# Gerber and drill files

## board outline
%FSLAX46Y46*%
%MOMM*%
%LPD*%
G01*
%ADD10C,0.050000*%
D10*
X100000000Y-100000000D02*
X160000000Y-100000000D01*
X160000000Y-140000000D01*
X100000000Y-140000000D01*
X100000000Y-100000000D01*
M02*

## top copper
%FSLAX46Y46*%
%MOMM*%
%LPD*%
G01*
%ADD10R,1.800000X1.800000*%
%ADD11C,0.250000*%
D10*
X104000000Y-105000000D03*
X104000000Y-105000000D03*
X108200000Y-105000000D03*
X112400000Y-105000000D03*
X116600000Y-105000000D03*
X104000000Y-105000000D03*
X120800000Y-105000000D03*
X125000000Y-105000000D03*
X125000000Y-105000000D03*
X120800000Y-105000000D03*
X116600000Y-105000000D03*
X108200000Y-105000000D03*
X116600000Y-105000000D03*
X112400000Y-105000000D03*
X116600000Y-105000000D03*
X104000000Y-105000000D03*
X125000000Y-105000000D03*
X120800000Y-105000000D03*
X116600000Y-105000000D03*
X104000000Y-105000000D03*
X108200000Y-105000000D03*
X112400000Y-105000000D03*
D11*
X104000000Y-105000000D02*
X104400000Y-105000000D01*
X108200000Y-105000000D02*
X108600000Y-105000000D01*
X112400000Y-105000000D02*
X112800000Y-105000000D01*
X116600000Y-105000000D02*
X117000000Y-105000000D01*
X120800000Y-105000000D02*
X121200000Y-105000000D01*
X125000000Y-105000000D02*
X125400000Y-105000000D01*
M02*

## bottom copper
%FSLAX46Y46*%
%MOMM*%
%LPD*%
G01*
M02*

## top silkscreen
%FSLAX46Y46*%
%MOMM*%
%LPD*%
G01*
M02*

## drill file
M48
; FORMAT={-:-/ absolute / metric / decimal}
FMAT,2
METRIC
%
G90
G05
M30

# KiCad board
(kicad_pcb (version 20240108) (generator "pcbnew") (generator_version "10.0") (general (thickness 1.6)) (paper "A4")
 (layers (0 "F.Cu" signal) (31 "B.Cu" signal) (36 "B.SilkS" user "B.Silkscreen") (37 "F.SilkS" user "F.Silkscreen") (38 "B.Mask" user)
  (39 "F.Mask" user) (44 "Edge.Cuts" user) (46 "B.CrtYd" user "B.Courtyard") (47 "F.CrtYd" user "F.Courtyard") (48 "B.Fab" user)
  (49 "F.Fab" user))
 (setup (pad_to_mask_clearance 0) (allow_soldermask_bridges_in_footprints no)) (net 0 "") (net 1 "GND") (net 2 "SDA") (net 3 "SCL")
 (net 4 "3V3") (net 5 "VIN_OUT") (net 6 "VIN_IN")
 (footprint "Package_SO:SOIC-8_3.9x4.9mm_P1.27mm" (layer "F.Cu") (at 100 100)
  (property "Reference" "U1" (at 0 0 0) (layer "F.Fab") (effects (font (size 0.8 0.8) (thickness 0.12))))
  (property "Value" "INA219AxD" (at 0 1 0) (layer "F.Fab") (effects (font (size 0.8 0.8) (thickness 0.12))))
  (pad "1" smd rect (at 4.000 5.000) (size 1.8 1.8) (layers "F.Cu" "F.Paste" "F.Mask") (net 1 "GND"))
  (pad "2" smd rect (at 4.000 5.000) (size 1.8 1.8) (layers "F.Cu" "F.Paste" "F.Mask") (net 1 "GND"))
  (pad "3" smd rect (at 8.200 5.000) (size 1.8 1.8) (layers "F.Cu" "F.Paste" "F.Mask") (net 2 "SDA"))
  (pad "4" smd rect (at 12.400 5.000) (size 1.8 1.8) (layers "F.Cu" "F.Paste" "F.Mask") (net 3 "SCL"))
  (pad "5" smd rect (at 16.600 5.000) (size 1.8 1.8) (layers "F.Cu" "F.Paste" "F.Mask") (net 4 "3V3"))
  (pad "6" smd rect (at 4.000 5.000) (size 1.8 1.8) (layers "F.Cu" "F.Paste" "F.Mask") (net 1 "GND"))
  (pad "7" smd rect (at 20.800 5.000) (size 1.8 1.8) (layers "F.Cu" "F.Paste" "F.Mask") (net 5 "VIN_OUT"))
  (pad "8" smd rect (at 25.000 5.000) (size 1.8 1.8) (layers "F.Cu" "F.Paste" "F.Mask") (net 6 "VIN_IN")))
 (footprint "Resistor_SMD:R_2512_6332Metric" (layer "F.Cu") (at 100 100)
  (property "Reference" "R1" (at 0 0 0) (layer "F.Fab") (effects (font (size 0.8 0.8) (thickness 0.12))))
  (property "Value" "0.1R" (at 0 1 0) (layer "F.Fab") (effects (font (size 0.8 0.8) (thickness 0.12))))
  (pad "1" smd rect (at 25.000 5.000) (size 1.8 1.8) (layers "F.Cu" "F.Paste" "F.Mask") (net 6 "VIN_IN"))
  (pad "2" smd rect (at 20.800 5.000) (size 1.8 1.8) (layers "F.Cu" "F.Paste" "F.Mask") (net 5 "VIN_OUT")))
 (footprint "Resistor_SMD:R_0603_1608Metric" (layer "F.Cu") (at 100 100)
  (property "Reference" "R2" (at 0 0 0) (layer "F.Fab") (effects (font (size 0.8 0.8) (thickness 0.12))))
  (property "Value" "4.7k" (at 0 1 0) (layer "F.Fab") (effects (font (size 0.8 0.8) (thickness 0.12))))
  (pad "1" smd rect (at 16.600 5.000) (size 1.8 1.8) (layers "F.Cu" "F.Paste" "F.Mask") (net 4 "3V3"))
  (pad "2" smd rect (at 8.200 5.000) (size 1.8 1.8) (layers "F.Cu" "F.Paste" "F.Mask") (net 2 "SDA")))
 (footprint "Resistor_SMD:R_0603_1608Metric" (layer "F.Cu") (at 100 100)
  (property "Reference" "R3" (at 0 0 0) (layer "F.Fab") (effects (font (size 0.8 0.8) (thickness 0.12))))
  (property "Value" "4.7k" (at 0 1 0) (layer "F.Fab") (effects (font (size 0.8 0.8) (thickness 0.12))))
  (pad "1" smd rect (at 16.600 5.000) (size 1.8 1.8) (layers "F.Cu" "F.Paste" "F.Mask") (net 4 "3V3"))
  (pad "2" smd rect (at 12.400 5.000) (size 1.8 1.8) (layers "F.Cu" "F.Paste" "F.Mask") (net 3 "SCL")))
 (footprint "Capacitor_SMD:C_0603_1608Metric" (layer "F.Cu") (at 100 100)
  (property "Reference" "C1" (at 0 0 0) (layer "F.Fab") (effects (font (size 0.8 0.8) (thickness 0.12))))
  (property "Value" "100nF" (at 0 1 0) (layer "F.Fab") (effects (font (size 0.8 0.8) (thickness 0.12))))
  (pad "1" smd rect (at 16.600 5.000) (size 1.8 1.8) (layers "F.Cu" "F.Paste" "F.Mask") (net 4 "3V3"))
  (pad "2" smd rect (at 4.000 5.000) (size 1.8 1.8) (layers "F.Cu" "F.Paste" "F.Mask") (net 1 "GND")))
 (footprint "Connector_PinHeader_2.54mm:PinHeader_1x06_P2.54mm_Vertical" (layer "F.Cu") (at 100 100)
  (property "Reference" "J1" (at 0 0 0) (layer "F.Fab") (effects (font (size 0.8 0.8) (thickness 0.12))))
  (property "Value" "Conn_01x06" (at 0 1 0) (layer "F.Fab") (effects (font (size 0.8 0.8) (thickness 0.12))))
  (pad "1" smd rect (at 25.000 5.000) (size 1.8 1.8) (layers "F.Cu" "F.Paste" "F.Mask") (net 6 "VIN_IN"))
  (pad "2" smd rect (at 20.800 5.000) (size 1.8 1.8) (layers "F.Cu" "F.Paste" "F.Mask") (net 5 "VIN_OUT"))
  (pad "3" smd rect (at 16.600 5.000) (size 1.8 1.8) (layers "F.Cu" "F.Paste" "F.Mask") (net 4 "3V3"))
  (pad "4" smd rect (at 4.000 5.000) (size 1.8 1.8) (layers "F.Cu" "F.Paste" "F.Mask") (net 1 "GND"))
  (pad "5" smd rect (at 8.200 5.000) (size 1.8 1.8) (layers "F.Cu" "F.Paste" "F.Mask") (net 2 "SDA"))
  (pad "6" smd rect (at 12.400 5.000) (size 1.8 1.8) (layers "F.Cu" "F.Paste" "F.Mask") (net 3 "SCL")))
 (gr_rect (start 100 100) (end 160 140) (stroke (width 0.05) (type default)) (fill none) (layer "Edge.Cuts"))
 (segment (start 104.000 105.000) (end 104.400 105.000) (width 0.25) (layer "F.Cu") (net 1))
 (segment (start 108.200 105.000) (end 108.600 105.000) (width 0.25) (layer "F.Cu") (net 2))
 (segment (start 112.400 105.000) (end 112.800 105.000) (width 0.25) (layer "F.Cu") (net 3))
 (segment (start 116.600 105.000) (end 117.000 105.000) (width 0.25) (layer "F.Cu") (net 4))
 (segment (start 120.800 105.000) (end 121.200 105.000) (width 0.25) (layer "F.Cu") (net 5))
 (segment (start 125.000 105.000) (end 125.400 105.000) (width 0.25) (layer "F.Cu") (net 6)))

